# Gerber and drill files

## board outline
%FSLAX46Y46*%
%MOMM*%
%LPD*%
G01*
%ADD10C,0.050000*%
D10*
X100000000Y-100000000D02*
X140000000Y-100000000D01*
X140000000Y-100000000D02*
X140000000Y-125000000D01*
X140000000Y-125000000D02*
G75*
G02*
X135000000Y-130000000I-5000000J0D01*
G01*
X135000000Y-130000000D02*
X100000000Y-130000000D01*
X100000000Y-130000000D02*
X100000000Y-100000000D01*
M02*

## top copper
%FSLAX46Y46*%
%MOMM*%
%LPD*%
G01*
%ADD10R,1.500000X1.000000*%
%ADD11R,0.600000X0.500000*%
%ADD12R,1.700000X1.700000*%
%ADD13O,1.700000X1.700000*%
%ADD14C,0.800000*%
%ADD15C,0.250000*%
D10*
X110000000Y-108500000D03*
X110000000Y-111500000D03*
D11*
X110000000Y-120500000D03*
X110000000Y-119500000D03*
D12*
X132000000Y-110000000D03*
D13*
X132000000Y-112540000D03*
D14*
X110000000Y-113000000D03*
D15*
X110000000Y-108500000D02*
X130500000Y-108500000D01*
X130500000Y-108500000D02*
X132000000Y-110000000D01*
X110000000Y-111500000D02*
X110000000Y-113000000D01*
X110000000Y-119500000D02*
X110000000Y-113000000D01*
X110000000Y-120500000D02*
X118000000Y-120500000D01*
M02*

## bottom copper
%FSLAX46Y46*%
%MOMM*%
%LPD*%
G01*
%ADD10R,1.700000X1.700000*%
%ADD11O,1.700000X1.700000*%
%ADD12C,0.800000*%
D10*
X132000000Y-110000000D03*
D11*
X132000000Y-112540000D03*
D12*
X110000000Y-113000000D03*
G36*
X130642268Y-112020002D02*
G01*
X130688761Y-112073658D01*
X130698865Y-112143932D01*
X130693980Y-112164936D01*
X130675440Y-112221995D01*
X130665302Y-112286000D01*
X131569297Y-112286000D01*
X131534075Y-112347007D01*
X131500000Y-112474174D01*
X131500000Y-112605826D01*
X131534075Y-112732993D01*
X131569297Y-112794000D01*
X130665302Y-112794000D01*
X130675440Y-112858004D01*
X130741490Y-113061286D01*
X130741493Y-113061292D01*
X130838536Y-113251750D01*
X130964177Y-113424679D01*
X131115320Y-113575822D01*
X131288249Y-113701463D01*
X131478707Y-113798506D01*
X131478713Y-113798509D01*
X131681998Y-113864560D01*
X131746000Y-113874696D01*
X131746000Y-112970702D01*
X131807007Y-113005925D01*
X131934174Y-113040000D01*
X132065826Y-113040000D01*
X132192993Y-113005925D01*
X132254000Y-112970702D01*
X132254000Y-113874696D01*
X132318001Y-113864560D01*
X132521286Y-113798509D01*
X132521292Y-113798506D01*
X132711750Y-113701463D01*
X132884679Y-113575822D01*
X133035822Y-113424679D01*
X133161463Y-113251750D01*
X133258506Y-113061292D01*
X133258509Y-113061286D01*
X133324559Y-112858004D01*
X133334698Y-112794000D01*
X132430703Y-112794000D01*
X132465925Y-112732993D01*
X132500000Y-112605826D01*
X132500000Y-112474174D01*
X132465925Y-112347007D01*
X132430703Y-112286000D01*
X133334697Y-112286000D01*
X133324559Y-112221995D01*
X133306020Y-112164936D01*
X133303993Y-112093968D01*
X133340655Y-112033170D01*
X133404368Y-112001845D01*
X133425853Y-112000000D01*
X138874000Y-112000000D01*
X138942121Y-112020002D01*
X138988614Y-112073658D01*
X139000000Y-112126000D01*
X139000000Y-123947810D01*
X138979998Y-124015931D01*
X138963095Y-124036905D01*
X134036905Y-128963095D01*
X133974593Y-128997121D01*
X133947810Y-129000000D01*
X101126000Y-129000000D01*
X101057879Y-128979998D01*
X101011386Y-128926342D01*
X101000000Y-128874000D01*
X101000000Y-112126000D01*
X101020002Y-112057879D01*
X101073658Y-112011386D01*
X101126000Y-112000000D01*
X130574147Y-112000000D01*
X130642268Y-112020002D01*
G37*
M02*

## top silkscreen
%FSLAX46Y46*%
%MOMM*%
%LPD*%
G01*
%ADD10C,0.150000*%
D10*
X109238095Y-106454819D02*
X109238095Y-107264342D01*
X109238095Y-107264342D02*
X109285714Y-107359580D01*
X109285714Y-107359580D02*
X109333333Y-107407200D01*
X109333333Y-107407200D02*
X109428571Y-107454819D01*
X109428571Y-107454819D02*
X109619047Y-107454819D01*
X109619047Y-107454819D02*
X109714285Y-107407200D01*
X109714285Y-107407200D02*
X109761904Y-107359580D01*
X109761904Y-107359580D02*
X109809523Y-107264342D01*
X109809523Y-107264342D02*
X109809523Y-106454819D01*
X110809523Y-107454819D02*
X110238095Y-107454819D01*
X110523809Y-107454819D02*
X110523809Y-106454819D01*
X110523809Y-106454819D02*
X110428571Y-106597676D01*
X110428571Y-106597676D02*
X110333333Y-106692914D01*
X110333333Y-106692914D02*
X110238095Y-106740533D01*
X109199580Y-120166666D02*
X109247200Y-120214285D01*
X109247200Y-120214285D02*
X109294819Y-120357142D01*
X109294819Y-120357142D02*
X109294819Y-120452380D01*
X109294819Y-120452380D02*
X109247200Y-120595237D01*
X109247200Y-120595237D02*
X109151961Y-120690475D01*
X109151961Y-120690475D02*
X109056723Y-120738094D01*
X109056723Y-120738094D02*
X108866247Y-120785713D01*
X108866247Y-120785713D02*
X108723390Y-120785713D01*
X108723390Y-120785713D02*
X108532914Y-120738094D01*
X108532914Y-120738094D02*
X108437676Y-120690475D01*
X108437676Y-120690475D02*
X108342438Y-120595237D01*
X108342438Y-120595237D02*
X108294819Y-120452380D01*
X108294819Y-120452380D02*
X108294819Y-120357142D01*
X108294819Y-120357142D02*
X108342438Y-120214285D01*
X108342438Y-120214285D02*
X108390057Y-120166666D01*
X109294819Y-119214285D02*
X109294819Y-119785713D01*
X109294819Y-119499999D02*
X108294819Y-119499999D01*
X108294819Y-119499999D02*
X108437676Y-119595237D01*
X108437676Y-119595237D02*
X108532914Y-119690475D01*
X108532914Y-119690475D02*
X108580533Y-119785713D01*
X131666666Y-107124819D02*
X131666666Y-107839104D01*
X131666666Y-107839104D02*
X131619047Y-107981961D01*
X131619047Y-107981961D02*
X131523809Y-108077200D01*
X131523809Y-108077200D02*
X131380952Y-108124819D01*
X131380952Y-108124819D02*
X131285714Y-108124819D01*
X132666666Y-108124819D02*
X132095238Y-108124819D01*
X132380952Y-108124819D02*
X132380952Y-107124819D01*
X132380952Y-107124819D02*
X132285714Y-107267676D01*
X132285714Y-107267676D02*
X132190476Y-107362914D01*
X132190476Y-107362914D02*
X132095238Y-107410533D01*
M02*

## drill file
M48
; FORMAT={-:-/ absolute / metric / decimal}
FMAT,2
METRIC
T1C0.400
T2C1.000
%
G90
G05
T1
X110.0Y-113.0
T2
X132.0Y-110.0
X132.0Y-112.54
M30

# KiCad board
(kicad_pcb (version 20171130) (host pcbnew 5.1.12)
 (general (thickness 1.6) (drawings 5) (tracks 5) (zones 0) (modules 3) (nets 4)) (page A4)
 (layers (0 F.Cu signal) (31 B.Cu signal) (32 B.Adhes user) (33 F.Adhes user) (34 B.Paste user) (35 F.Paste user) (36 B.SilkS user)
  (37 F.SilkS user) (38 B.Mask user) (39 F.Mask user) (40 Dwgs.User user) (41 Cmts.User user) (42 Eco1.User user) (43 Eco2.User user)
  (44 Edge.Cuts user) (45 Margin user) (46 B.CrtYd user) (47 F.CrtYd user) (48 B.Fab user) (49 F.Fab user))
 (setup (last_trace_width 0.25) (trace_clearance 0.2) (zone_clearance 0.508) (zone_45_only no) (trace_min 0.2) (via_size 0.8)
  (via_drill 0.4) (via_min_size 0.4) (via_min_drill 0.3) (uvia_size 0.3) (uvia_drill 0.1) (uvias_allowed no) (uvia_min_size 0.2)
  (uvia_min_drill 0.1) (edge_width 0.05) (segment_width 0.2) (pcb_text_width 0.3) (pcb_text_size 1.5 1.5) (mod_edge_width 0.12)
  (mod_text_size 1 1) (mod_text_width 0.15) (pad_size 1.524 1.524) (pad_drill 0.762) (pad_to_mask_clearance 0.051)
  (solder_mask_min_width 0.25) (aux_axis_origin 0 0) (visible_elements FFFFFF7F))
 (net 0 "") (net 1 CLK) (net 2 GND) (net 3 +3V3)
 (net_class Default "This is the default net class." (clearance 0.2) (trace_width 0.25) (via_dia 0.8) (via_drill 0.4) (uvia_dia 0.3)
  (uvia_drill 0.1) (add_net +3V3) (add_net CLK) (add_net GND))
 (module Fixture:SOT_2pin (layer F.Cu) (at 110 110)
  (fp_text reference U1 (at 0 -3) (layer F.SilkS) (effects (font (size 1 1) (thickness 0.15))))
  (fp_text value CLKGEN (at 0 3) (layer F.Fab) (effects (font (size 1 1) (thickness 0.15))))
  (pad 1 smd rect (at 0 -1.5) (size 1.5 1) (layers F.Cu F.Paste F.Mask) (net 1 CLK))
  (pad 2 smd rect (at 0 1.5) (size 1.5 1) (layers F.Cu F.Paste F.Mask) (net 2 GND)))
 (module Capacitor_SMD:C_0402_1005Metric (layer F.Cu) (at 110 120 90)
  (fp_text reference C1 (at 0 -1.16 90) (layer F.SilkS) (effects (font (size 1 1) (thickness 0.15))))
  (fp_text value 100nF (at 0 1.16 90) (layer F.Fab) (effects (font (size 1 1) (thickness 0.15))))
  (pad 1 smd rect (at -0.5 0 90) (size 0.5 0.6) (layers F.Cu F.Paste F.Mask) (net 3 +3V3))
  (pad 2 smd rect (at 0.5 0 90) (size 0.5 0.6) (layers F.Cu F.Paste F.Mask) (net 2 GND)))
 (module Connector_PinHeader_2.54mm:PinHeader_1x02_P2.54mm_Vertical (layer F.Cu) (at 132 110)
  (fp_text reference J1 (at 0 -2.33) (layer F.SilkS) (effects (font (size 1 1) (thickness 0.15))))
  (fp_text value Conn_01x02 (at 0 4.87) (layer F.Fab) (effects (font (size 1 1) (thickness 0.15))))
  (pad 1 thru_hole rect (at 0 0) (size 1.7 1.7) (drill 1) (layers *.Cu *.Mask) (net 1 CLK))
  (pad 2 thru_hole oval (at 0 2.54) (size 1.7 1.7) (drill 1) (layers *.Cu *.Mask) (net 2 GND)))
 (gr_line (start 100 100) (end 140 100) (layer Edge.Cuts) (width 0.05))
 (gr_line (start 140 100) (end 140 125) (layer Edge.Cuts) (width 0.05))
 (gr_arc (start 135 125) (end 140 125) (angle 90) (layer Edge.Cuts) (width 0.05))
 (gr_line (start 135 130) (end 100 130) (layer Edge.Cuts) (width 0.05))
 (gr_line (start 100 130) (end 100 100) (layer Edge.Cuts) (width 0.05))
 (segment (start 110 108.5) (end 130.5 108.5) (width 0.25) (layer F.Cu) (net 1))
 (segment (start 130.5 108.5) (end 132 110) (width 0.25) (layer F.Cu) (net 1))
 (segment (start 110 111.5) (end 110 113) (width 0.25) (layer F.Cu) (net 2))
 (segment (start 110 119.5) (end 110 113) (width 0.25) (layer F.Cu) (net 2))
 (segment (start 110 120.5) (end 118 120.5) (width 0.25) (layer F.Cu) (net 3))
 (via (at 110 113) (size 0.8) (drill 0.4) (layers F.Cu B.Cu) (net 2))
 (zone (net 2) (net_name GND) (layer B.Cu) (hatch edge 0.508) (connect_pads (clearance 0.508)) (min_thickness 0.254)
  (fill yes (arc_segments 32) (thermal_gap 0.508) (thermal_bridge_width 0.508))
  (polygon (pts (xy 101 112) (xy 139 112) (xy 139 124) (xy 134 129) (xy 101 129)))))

